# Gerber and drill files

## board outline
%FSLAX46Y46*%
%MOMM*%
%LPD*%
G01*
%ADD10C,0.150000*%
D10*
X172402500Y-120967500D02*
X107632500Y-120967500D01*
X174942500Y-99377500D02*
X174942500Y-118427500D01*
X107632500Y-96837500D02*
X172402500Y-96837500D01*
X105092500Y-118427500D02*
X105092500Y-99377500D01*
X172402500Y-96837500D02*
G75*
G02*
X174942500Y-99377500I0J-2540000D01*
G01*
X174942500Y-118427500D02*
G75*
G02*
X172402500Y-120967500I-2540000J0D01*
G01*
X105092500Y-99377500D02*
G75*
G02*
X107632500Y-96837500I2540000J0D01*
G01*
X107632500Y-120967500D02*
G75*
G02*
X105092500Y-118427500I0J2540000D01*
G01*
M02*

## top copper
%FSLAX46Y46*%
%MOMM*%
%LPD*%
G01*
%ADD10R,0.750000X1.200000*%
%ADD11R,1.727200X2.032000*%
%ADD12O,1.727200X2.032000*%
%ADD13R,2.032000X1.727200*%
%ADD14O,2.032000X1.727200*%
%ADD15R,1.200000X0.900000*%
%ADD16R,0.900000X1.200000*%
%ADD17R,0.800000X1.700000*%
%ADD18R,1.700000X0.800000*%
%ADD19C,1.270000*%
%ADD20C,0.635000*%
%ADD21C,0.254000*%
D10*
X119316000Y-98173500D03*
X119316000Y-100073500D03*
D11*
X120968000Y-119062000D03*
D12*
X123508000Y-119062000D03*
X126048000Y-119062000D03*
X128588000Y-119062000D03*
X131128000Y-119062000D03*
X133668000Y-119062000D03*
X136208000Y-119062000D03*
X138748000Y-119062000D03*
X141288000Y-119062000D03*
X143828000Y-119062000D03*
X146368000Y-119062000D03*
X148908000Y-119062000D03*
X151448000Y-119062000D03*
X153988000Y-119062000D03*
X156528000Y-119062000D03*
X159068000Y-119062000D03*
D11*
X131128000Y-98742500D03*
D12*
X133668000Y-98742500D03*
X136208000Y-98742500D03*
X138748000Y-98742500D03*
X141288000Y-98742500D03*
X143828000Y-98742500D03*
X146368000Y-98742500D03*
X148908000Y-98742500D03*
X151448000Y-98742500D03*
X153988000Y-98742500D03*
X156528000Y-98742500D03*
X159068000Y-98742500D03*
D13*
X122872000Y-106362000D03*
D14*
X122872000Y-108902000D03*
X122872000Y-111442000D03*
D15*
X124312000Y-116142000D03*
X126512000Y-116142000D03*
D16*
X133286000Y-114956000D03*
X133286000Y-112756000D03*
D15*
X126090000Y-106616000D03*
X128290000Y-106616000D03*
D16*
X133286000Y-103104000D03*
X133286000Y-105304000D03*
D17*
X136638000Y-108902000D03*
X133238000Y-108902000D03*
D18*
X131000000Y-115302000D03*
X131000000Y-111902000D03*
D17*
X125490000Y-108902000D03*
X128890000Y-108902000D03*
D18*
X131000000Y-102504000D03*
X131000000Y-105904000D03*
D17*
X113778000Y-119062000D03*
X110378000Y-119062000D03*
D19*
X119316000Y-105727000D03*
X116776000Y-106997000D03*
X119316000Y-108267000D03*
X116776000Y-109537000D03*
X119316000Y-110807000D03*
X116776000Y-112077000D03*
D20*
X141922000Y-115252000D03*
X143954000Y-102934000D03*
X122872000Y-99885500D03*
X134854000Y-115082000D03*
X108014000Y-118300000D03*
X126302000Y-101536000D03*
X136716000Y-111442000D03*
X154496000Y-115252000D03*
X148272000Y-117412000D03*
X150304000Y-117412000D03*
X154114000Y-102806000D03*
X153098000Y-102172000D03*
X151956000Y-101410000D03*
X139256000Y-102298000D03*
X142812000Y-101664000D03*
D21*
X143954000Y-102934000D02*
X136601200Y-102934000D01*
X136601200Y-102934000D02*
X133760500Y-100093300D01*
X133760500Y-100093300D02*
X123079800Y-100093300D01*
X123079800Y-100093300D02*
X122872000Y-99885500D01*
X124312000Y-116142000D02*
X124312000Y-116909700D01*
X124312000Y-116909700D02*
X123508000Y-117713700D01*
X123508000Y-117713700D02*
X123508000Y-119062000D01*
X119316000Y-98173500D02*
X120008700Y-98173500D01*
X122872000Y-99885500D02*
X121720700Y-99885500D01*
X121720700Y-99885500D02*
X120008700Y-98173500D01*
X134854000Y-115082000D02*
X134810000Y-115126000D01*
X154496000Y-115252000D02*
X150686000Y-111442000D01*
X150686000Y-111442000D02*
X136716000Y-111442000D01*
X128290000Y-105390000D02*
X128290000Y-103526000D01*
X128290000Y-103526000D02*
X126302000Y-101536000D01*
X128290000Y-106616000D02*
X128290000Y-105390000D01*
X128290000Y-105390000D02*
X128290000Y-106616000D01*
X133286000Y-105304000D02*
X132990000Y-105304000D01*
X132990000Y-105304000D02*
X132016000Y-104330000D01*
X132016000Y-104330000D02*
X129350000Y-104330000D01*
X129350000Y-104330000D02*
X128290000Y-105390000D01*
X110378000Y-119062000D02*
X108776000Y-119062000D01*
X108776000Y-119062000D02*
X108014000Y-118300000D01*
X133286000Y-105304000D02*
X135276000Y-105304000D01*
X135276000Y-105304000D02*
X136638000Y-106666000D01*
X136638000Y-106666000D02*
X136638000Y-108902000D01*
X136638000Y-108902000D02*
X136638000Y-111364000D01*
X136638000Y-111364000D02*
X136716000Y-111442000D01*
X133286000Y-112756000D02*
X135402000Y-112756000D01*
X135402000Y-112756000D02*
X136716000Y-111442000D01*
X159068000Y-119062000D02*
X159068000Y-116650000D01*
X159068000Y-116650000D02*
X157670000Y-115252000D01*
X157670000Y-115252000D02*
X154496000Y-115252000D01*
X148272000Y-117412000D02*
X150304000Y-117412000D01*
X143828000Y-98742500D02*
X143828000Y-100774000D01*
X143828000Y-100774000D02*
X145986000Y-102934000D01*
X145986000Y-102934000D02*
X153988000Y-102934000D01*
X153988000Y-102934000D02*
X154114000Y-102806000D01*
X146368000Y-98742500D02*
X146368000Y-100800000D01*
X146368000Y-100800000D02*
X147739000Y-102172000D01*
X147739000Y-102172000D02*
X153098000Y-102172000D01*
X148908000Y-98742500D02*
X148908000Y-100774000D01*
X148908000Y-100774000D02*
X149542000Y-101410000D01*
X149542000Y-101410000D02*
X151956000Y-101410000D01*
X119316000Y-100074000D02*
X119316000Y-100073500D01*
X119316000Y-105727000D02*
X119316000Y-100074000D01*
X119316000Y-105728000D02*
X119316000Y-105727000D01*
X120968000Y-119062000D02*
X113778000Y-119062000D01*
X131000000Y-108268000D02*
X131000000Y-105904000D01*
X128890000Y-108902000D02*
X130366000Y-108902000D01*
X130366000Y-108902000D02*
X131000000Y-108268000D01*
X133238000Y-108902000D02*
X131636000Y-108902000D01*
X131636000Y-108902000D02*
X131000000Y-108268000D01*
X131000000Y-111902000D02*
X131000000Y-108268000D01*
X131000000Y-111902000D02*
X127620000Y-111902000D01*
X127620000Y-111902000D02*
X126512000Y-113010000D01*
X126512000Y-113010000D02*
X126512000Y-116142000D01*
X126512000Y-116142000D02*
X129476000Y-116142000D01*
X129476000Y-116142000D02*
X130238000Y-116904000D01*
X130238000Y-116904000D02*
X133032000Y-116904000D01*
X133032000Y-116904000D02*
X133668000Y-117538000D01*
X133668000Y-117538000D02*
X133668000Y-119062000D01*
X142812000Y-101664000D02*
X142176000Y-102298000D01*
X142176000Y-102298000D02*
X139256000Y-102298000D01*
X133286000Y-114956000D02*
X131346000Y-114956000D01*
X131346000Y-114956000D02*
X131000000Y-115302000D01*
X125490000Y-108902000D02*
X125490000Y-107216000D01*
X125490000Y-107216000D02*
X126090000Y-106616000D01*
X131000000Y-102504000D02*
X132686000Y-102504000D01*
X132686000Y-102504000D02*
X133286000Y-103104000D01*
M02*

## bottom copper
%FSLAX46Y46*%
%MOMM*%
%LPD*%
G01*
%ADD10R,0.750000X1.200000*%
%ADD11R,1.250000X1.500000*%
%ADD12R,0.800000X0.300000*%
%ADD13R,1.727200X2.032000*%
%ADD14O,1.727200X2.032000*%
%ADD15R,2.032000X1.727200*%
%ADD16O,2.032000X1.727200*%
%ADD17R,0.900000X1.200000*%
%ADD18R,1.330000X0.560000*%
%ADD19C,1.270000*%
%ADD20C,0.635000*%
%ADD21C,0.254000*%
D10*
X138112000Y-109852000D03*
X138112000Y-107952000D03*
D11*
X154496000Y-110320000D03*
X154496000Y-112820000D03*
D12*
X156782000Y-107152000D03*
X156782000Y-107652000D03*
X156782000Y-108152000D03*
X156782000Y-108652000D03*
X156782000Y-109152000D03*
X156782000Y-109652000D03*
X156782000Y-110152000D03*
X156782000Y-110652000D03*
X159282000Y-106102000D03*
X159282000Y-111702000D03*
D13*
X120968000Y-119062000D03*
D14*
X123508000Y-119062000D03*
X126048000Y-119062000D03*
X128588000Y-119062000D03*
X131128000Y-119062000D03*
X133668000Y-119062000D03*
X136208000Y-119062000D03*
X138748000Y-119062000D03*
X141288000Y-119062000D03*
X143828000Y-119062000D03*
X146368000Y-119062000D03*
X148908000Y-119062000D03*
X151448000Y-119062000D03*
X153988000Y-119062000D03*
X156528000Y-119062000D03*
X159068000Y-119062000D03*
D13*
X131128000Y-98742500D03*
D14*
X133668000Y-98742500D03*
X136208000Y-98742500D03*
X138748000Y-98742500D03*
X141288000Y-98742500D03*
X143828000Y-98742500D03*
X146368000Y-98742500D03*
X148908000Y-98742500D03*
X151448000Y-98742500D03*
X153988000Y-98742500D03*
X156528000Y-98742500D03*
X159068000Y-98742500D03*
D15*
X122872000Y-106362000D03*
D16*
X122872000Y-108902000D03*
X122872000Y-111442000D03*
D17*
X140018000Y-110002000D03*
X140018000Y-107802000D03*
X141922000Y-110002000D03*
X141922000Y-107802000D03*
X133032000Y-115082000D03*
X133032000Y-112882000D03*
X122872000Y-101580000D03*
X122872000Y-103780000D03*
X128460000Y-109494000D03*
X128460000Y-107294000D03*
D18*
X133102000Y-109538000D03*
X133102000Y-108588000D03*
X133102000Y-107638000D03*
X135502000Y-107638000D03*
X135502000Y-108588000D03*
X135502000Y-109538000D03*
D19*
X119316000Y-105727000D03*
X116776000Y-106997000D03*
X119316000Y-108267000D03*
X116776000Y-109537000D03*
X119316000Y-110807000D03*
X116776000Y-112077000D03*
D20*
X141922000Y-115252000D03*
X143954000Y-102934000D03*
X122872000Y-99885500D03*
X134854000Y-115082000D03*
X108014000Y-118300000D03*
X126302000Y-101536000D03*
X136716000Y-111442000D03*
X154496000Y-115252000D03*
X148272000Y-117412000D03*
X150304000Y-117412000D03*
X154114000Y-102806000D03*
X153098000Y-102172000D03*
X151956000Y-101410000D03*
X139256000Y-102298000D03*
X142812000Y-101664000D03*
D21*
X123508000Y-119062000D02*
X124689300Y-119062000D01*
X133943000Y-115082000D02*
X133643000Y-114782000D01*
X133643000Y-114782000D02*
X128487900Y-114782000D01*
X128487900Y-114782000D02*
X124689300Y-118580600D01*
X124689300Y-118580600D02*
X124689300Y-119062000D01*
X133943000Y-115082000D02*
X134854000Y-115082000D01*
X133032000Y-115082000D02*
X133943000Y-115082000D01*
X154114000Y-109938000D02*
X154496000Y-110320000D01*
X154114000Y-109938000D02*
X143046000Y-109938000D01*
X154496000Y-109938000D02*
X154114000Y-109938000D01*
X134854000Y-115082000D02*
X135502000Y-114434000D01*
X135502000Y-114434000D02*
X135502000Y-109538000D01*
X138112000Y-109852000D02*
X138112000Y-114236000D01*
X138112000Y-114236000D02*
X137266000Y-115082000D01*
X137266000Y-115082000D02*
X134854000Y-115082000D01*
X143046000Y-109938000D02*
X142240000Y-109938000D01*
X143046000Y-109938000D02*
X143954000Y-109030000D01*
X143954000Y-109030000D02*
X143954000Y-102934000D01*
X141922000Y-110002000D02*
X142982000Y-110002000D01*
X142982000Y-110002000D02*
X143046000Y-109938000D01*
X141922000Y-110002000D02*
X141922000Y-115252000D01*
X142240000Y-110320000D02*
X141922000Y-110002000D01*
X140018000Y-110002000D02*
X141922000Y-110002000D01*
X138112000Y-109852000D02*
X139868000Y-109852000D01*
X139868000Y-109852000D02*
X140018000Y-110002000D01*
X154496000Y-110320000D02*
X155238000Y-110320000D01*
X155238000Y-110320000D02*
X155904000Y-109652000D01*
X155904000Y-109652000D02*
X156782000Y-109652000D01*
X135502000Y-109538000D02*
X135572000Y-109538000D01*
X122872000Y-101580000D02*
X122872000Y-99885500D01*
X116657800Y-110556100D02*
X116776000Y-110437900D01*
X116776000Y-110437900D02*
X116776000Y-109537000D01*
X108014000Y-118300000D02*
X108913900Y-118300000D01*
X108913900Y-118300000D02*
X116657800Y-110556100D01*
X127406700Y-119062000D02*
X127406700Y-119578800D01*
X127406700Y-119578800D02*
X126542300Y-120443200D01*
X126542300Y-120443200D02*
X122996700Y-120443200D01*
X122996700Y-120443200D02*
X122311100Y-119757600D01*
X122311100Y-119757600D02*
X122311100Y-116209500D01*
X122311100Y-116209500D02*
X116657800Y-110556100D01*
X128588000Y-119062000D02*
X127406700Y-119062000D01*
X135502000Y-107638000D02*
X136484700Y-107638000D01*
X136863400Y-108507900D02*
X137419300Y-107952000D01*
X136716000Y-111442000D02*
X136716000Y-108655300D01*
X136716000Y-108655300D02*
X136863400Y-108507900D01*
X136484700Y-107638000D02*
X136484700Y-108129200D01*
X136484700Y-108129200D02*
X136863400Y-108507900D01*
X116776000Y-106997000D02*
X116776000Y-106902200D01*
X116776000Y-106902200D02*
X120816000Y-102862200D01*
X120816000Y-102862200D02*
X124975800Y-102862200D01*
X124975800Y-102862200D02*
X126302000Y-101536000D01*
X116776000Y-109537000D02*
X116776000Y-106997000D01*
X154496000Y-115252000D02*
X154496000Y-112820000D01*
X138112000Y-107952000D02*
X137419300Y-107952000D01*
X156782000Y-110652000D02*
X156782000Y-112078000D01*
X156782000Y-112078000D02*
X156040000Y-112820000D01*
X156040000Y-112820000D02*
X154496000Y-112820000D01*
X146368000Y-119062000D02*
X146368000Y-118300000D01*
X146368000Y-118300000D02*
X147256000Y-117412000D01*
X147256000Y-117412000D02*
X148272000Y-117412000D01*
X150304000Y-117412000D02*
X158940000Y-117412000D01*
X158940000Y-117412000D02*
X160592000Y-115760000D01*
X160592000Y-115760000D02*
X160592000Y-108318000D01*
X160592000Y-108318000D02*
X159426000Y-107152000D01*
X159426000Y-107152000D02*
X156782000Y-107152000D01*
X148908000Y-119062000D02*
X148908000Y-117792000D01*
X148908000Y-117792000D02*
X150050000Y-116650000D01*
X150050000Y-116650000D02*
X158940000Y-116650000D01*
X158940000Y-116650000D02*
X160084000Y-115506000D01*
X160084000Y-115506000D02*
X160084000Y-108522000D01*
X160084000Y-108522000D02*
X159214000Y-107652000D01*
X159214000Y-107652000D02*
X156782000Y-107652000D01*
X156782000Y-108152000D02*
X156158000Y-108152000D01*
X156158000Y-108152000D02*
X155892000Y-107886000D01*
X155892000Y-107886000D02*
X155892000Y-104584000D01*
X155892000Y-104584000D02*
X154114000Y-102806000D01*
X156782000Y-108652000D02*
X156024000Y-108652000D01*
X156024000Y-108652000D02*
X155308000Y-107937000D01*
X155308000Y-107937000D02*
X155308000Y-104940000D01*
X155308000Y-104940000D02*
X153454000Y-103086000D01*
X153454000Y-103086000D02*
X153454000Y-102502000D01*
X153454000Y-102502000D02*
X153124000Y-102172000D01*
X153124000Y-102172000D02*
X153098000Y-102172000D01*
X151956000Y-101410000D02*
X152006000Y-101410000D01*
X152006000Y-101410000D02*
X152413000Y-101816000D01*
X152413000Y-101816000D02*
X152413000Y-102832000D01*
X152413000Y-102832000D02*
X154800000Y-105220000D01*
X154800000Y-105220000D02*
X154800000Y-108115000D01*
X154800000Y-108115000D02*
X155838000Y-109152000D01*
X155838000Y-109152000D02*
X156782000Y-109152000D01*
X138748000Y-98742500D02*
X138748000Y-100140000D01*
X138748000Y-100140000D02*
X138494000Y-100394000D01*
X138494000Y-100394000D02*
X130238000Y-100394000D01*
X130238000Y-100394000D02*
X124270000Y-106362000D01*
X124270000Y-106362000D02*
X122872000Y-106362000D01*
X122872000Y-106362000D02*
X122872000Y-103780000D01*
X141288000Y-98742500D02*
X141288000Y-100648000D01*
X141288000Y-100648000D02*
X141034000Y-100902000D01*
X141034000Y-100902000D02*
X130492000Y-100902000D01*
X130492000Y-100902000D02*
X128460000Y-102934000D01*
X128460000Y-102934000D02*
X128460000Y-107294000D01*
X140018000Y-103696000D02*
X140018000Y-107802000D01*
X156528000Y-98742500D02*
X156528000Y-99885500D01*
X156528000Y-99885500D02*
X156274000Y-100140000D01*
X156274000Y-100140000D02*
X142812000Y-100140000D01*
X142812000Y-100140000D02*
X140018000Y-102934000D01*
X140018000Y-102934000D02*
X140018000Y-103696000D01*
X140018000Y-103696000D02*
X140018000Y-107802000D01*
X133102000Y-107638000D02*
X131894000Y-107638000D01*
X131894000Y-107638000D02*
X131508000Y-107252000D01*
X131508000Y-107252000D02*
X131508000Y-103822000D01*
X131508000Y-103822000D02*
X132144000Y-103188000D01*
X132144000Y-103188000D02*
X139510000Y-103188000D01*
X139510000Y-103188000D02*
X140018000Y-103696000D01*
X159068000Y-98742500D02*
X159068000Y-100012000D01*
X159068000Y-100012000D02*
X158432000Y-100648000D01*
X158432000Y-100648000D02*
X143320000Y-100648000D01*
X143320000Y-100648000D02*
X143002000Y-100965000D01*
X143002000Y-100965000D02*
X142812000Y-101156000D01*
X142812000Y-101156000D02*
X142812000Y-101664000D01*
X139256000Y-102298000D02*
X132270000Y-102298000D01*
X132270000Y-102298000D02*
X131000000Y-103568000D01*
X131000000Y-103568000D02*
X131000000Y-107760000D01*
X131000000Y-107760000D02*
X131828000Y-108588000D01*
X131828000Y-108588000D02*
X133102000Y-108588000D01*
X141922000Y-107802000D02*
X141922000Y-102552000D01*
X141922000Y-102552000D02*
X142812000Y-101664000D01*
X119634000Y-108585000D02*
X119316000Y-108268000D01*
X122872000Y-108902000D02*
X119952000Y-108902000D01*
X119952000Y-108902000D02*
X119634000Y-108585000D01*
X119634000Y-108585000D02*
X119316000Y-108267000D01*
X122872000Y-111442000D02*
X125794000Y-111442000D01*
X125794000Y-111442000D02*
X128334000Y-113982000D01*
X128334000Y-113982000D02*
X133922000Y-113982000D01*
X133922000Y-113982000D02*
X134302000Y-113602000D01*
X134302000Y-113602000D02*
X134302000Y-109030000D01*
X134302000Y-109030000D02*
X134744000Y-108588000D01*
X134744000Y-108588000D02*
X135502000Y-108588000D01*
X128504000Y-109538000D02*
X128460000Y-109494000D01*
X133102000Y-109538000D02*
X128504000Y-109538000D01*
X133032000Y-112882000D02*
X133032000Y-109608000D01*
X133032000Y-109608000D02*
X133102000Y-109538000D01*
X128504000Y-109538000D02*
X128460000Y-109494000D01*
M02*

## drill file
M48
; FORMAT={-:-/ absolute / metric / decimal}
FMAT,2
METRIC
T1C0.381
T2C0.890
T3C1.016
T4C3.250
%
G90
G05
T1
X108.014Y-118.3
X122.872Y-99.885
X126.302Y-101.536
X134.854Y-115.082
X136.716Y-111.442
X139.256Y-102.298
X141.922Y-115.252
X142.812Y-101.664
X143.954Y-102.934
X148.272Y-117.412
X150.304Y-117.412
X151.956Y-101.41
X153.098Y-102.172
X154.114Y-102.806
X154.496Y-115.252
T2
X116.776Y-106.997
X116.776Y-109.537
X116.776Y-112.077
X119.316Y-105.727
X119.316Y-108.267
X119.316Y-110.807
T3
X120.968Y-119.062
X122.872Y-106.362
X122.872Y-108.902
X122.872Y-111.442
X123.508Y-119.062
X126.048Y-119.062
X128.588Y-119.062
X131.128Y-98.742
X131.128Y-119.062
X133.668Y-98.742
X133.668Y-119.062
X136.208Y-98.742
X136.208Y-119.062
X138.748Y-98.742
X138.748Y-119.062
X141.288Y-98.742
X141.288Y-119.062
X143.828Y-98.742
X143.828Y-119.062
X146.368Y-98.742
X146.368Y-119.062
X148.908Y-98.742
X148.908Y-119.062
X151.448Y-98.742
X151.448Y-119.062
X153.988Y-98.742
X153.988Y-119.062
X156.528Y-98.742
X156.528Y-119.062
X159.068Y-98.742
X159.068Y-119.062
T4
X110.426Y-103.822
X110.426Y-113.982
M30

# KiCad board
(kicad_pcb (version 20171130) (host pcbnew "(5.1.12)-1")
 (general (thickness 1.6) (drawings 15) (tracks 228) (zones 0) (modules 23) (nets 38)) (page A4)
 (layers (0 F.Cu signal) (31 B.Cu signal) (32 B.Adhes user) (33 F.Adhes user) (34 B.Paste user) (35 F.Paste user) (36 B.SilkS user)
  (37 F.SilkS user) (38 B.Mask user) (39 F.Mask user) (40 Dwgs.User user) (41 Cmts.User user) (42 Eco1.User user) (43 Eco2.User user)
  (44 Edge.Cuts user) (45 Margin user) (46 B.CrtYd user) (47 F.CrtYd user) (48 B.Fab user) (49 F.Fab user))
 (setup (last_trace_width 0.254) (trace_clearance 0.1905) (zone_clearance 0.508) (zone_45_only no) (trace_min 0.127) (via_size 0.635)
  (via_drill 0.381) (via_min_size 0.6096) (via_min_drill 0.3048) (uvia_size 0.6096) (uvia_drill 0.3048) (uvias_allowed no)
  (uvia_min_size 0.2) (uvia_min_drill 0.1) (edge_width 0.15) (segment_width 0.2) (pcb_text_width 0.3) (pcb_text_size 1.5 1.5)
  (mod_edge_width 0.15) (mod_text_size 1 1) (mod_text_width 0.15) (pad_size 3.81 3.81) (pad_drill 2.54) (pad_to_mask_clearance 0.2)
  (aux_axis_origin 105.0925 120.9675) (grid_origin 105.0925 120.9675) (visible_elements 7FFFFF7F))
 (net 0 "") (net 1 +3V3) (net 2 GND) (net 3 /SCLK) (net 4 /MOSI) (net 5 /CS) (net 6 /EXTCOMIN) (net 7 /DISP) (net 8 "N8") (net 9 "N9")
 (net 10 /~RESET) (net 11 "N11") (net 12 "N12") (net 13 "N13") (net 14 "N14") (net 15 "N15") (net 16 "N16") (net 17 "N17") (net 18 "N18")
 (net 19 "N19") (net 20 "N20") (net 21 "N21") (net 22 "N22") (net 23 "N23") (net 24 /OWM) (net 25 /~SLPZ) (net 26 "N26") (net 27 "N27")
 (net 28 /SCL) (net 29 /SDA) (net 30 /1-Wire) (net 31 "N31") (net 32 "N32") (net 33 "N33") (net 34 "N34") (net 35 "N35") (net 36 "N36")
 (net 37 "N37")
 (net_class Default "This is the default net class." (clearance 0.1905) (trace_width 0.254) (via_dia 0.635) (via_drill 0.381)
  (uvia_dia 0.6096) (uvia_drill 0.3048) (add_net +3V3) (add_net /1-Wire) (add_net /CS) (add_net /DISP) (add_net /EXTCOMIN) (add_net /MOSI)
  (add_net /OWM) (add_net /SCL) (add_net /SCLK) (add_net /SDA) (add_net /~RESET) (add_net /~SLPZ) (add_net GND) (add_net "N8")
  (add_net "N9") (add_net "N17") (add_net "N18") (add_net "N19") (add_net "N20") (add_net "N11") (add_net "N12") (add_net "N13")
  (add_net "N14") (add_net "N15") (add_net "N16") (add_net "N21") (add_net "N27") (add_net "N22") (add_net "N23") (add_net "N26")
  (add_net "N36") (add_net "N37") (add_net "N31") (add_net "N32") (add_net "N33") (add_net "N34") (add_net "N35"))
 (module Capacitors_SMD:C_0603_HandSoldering (layer B.Cu) (at 138.112 108.902 90)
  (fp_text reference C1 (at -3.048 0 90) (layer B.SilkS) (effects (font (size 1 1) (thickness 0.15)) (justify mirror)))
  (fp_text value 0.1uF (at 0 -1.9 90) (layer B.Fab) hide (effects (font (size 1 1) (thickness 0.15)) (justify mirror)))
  (pad 1 smd rect (at -0.95 0 90) (size 1.2 0.75) (layers B.Cu B.Paste B.Mask) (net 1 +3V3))
  (pad 2 smd rect (at 0.95 0 90) (size 1.2 0.75) (layers B.Cu B.Paste B.Mask) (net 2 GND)))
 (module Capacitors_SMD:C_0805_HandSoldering (layer B.Cu) (at 154.496 111.57 270)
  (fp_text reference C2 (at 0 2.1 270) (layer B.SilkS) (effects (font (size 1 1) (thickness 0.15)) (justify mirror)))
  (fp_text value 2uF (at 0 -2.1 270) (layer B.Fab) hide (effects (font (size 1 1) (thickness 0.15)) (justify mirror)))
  (pad 1 smd rect (at -1.25 0 270) (size 1.5 1.25) (layers B.Cu B.Paste B.Mask) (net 1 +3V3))
  (pad 2 smd rect (at 1.25 0 270) (size 1.5 1.25) (layers B.Cu B.Paste B.Mask) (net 2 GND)))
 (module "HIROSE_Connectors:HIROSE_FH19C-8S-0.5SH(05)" (layer B.Cu) (at 156.782 108.902 270)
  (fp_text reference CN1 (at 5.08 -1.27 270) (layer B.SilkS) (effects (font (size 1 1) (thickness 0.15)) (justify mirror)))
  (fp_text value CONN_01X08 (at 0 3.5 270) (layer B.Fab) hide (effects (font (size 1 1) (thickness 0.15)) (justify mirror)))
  (pad 1 smd rect (at -1.75 0 270) (size 0.3 0.8) (layers B.Cu B.Paste B.Mask) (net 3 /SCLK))
  (pad 2 smd rect (at -1.25 0 270) (size 0.3 0.8) (layers B.Cu B.Paste B.Mask) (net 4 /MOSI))
  (pad 3 smd rect (at -0.75 0 270) (size 0.3 0.8) (layers B.Cu B.Paste B.Mask) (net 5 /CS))
  (pad 4 smd rect (at -0.25 0 270) (size 0.3 0.8) (layers B.Cu B.Paste B.Mask) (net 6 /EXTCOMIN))
  (pad 5 smd rect (at 0.25 0 270) (size 0.3 0.8) (layers B.Cu B.Paste B.Mask) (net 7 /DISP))
  (pad 6 smd rect (at 0.75 0 270) (size 0.3 0.8) (layers B.Cu B.Paste B.Mask) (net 1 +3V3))
  (pad 7 smd rect (at 1.25 0 270) (size 0.3 0.8) (layers B.Cu B.Paste B.Mask) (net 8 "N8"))
  (pad 8 smd rect (at 1.75 0 270) (size 0.3 0.8) (layers B.Cu B.Paste B.Mask) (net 2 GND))
  (pad "" smd rect (at -2.8 -2.5 270) (size 0.3 0.8) (layers B.Cu B.Paste B.Mask))
  (pad "" smd rect (at 2.8 -2.5 270) (size 0.3 0.8) (layers B.Cu B.Paste B.Mask)))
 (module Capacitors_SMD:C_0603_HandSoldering (layer F.Cu) (at 119.316 99.1235 270)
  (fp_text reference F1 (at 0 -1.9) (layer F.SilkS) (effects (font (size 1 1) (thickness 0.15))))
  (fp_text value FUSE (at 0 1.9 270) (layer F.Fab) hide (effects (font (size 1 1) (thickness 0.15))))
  (pad 1 smd rect (at -0.95 0 270) (size 1.2 0.75) (layers F.Cu F.Paste F.Mask) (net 1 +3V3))
  (pad 2 smd rect (at 0.95 0 270) (size 1.2 0.75) (layers F.Cu F.Paste F.Mask) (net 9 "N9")))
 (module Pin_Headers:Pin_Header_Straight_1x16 (layer B.Cu) (at 120.968 119.062 270)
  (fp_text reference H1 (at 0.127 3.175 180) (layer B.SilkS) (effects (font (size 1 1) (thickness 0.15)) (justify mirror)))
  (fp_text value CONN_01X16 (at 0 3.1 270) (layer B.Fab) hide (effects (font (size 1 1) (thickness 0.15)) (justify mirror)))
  (pad 1 thru_hole rect (at 0 0 270) (size 2.032 1.7272) (drill 1.016) (layers *.Cu *.Mask B.SilkS) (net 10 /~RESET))
  (pad 2 thru_hole oval (at 0 -2.54 270) (size 2.032 1.7272) (drill 1.016) (layers *.Cu *.Mask B.SilkS) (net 1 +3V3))
  (pad 3 thru_hole oval (at 0 -5.08 270) (size 2.032 1.7272) (drill 1.016) (layers *.Cu *.Mask B.SilkS) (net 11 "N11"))
  (pad 4 thru_hole oval (at 0 -7.62 270) (size 2.032 1.7272) (drill 1.016) (layers *.Cu *.Mask B.SilkS) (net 2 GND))
  (pad 5 thru_hole oval (at 0 -10.16 270) (size 2.032 1.7272) (drill 1.016) (layers *.Cu *.Mask B.SilkS) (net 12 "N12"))
  (pad 6 thru_hole oval (at 0 -12.7 270) (size 2.032 1.7272) (drill 1.016) (layers *.Cu *.Mask B.SilkS) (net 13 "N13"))
  (pad 7 thru_hole oval (at 0 -15.24 270) (size 2.032 1.7272) (drill 1.016) (layers *.Cu *.Mask B.SilkS) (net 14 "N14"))
  (pad 8 thru_hole oval (at 0 -17.78 270) (size 2.032 1.7272) (drill 1.016) (layers *.Cu *.Mask B.SilkS) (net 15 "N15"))
  (pad 9 thru_hole oval (at 0 -20.32 270) (size 2.032 1.7272) (drill 1.016) (layers *.Cu *.Mask B.SilkS) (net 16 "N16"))
  (pad 10 thru_hole oval (at 0 -22.86 270) (size 2.032 1.7272) (drill 1.016) (layers *.Cu *.Mask B.SilkS) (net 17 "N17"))
  (pad 11 thru_hole oval (at 0 -25.4 270) (size 2.032 1.7272) (drill 1.016) (layers *.Cu *.Mask B.SilkS) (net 3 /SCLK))
  (pad 12 thru_hole oval (at 0 -27.94 270) (size 2.032 1.7272) (drill 1.016) (layers *.Cu *.Mask B.SilkS) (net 4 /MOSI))
  (pad 13 thru_hole oval (at 0 -30.48 270) (size 2.032 1.7272) (drill 1.016) (layers *.Cu *.Mask B.SilkS) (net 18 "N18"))
  (pad 14 thru_hole oval (at 0 -33.02 270) (size 2.032 1.7272) (drill 1.016) (layers *.Cu *.Mask B.SilkS) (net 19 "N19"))
  (pad 15 thru_hole oval (at 0 -35.56 270) (size 2.032 1.7272) (drill 1.016) (layers *.Cu *.Mask B.SilkS) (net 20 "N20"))
  (pad 16 thru_hole oval (at 0 -38.1 270) (size 2.032 1.7272) (drill 1.016) (layers *.Cu *.Mask B.SilkS) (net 2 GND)))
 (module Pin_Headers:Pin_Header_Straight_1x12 (layer B.Cu) (at 131.128 98.7425 270)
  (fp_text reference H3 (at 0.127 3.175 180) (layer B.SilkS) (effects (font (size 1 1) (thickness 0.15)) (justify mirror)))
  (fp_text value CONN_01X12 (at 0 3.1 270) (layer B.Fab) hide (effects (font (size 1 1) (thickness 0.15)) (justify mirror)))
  (pad 1 thru_hole rect (at 0 0 270) (size 2.032 1.7272) (drill 1.016) (layers *.Cu *.Mask B.SilkS) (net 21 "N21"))
  (pad 2 thru_hole oval (at 0 -2.54 270) (size 2.032 1.7272) (drill 1.016) (layers *.Cu *.Mask B.SilkS) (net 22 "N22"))
  (pad 3 thru_hole oval (at 0 -5.08 270) (size 2.032 1.7272) (drill 1.016) (layers *.Cu *.Mask B.SilkS) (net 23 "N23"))
  (pad 4 thru_hole oval (at 0 -7.62 270) (size 2.032 1.7272) (drill 1.016) (layers *.Cu *.Mask B.SilkS) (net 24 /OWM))
  (pad 5 thru_hole oval (at 0 -10.16 270) (size 2.032 1.7272) (drill 1.016) (layers *.Cu *.Mask B.SilkS) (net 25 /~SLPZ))
  (pad 6 thru_hole oval (at 0 -12.7 270) (size 2.032 1.7272) (drill 1.016) (layers *.Cu *.Mask B.SilkS) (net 5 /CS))
  (pad 7 thru_hole oval (at 0 -15.24 270) (size 2.032 1.7272) (drill 1.016) (layers *.Cu *.Mask B.SilkS) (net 6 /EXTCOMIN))
  (pad 8 thru_hole oval (at 0 -17.78 270) (size 2.032 1.7272) (drill 1.016) (layers *.Cu *.Mask B.SilkS) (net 7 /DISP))
  (pad 9 thru_hole oval (at 0 -20.32 270) (size 2.032 1.7272) (drill 1.016) (layers *.Cu *.Mask B.SilkS) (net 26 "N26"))
  (pad 10 thru_hole oval (at 0 -22.86 270) (size 2.032 1.7272) (drill 1.016) (layers *.Cu *.Mask B.SilkS) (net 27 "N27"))
  (pad 11 thru_hole oval (at 0 -25.4 270) (size 2.032 1.7272) (drill 1.016) (layers *.Cu *.Mask B.SilkS) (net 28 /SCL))
  (pad 12 thru_hole oval (at 0 -27.94 270) (size 2.032 1.7272) (drill 1.016) (layers *.Cu *.Mask B.SilkS) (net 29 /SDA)))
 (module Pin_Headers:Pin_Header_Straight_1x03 (layer F.Cu) (at 122.872 106.362)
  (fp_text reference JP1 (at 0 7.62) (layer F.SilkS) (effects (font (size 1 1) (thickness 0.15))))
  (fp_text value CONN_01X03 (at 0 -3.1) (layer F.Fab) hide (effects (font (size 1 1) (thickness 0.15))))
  (pad 1 thru_hole rect (at 0 0) (size 2.032 1.7272) (drill 1.016) (layers *.Cu *.Mask F.SilkS) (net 24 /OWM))
  (pad 2 thru_hole oval (at 0 2.54) (size 2.032 1.7272) (drill 1.016) (layers *.Cu *.Mask F.SilkS) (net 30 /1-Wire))
  (pad 3 thru_hole oval (at 0 5.08) (size 2.032 1.7272) (drill 1.016) (layers *.Cu *.Mask F.SilkS) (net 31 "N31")))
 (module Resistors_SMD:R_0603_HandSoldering (layer B.Cu) (at 140.018 108.902 90)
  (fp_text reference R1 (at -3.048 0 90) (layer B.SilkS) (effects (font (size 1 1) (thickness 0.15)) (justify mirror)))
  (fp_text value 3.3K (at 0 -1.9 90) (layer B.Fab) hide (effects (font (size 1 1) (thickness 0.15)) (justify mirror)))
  (pad 1 smd rect (at -1.1 0 90) (size 1.2 0.9) (layers B.Cu B.Paste B.Mask) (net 1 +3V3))
  (pad 2 smd rect (at 1.1 0 90) (size 1.2 0.9) (layers B.Cu B.Paste B.Mask) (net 28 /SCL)))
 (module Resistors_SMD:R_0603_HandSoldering (layer B.Cu) (at 141.922 108.902 90)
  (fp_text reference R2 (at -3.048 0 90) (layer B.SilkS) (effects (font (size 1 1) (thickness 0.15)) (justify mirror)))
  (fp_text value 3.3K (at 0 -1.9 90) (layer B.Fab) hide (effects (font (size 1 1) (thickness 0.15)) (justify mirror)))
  (pad 1 smd rect (at -1.1 0 90) (size 1.2 0.9) (layers B.Cu B.Paste B.Mask) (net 1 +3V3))
  (pad 2 smd rect (at 1.1 0 90) (size 1.2 0.9) (layers B.Cu B.Paste B.Mask) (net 29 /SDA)))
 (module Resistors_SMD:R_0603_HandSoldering (layer B.Cu) (at 133.032 113.982 90)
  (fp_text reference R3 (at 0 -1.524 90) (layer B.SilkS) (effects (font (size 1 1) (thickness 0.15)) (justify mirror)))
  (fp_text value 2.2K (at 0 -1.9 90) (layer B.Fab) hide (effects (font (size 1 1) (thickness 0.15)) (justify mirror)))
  (pad 1 smd rect (at -1.1 0 90) (size 1.2 0.9) (layers B.Cu B.Paste B.Mask) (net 1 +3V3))
  (pad 2 smd rect (at 1.1 0 90) (size 1.2 0.9) (layers B.Cu B.Paste B.Mask) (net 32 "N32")))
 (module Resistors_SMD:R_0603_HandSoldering (layer B.Cu) (at 122.872 102.68 270)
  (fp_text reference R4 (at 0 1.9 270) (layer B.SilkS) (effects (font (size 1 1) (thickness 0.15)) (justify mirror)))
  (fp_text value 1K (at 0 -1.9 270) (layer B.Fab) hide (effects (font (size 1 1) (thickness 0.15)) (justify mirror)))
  (pad 1 smd rect (at -1.1 0 270) (size 1.2 0.9) (layers B.Cu B.Paste B.Mask) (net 1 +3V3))
  (pad 2 smd rect (at 1.1 0 270) (size 1.2 0.9) (layers B.Cu B.Paste B.Mask) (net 24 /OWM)))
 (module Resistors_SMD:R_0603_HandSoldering (layer B.Cu) (at 128.46 108.394 90)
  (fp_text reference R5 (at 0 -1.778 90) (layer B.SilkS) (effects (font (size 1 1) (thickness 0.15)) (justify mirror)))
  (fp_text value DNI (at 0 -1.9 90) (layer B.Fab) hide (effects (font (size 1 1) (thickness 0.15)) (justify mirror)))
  (pad 1 smd rect (at -1.1 0 90) (size 1.2 0.9) (layers B.Cu B.Paste B.Mask) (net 32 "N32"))
  (pad 2 smd rect (at 1.1 0 90) (size 1.2 0.9) (layers B.Cu B.Paste B.Mask) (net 25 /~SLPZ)))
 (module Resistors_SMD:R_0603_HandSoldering (layer F.Cu) (at 125.412 116.142)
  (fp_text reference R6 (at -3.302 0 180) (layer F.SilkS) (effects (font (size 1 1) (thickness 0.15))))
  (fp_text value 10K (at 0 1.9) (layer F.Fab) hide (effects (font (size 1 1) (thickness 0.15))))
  (pad 1 smd rect (at -1.1 0) (size 1.2 0.9) (layers F.Cu F.Paste F.Mask) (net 1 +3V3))
  (pad 2 smd rect (at 1.1 0) (size 1.2 0.9) (layers F.Cu F.Paste F.Mask) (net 13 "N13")))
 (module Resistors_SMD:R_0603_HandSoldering (layer F.Cu) (at 133.286 113.856 90)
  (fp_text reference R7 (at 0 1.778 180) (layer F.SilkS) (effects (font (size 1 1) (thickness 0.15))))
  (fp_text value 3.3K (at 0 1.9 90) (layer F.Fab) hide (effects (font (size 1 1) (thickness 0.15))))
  (pad 1 smd rect (at -1.1 0 90) (size 1.2 0.9) (layers F.Cu F.Paste F.Mask) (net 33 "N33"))
  (pad 2 smd rect (at 1.1 0 90) (size 1.2 0.9) (layers F.Cu F.Paste F.Mask) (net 2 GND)))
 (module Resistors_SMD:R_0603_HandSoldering (layer F.Cu) (at 127.19 106.616)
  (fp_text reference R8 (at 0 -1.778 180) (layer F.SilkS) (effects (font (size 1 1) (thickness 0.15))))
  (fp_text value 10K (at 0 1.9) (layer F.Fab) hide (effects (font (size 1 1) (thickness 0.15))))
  (pad 1 smd rect (at -1.1 0) (size 1.2 0.9) (layers F.Cu F.Paste F.Mask) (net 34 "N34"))
  (pad 2 smd rect (at 1.1 0) (size 1.2 0.9) (layers F.Cu F.Paste F.Mask) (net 2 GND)))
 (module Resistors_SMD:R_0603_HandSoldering (layer F.Cu) (at 133.286 104.204 270)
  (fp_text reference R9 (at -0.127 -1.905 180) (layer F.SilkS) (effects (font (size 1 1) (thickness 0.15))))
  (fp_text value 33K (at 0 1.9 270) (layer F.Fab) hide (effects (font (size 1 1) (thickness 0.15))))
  (pad 1 smd rect (at -1.1 0 270) (size 1.2 0.9) (layers F.Cu F.Paste F.Mask) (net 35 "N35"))
  (pad 2 smd rect (at 1.1 0 270) (size 1.2 0.9) (layers F.Cu F.Paste F.Mask) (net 2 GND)))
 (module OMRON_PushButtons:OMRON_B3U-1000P (layer F.Cu) (at 134.938 108.902 180)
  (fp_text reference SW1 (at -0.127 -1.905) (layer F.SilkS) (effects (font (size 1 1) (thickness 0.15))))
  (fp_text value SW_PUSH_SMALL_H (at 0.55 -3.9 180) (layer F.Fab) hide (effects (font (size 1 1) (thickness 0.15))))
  (pad 1 smd rect (at -1.7 0 180) (size 0.8 1.7) (layers F.Cu F.Paste F.Mask) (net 2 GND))
  (pad 2 smd rect (at 1.7 0 180) (size 0.8 1.7) (layers F.Cu F.Paste F.Mask) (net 13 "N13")))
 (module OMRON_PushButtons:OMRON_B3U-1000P (layer F.Cu) (at 131 113.602 90)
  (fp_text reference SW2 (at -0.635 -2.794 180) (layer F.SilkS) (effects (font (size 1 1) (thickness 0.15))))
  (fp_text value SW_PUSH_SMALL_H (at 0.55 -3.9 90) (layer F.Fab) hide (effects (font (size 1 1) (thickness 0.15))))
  (pad 1 smd rect (at -1.7 0 90) (size 0.8 1.7) (layers F.Cu F.Paste F.Mask) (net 33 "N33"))
  (pad 2 smd rect (at 1.7 0 90) (size 0.8 1.7) (layers F.Cu F.Paste F.Mask) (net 13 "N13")))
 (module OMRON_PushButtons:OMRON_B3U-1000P (layer F.Cu) (at 127.19 108.902)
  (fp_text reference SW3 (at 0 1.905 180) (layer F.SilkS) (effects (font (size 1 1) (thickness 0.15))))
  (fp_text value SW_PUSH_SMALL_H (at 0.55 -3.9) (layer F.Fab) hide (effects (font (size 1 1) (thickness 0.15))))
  (pad 1 smd rect (at -1.7 0) (size 0.8 1.7) (layers F.Cu F.Paste F.Mask) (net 34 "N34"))
  (pad 2 smd rect (at 1.7 0) (size 0.8 1.7) (layers F.Cu F.Paste F.Mask) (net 13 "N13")))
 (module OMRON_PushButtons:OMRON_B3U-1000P (layer F.Cu) (at 131 104.204 270)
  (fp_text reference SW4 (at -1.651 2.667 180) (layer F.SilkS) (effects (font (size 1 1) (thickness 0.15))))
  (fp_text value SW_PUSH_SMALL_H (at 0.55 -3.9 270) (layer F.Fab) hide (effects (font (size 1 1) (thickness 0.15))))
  (pad 1 smd rect (at -1.7 0 270) (size 0.8 1.7) (layers F.Cu F.Paste F.Mask) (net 35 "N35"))
  (pad 2 smd rect (at 1.7 0 270) (size 0.8 1.7) (layers F.Cu F.Paste F.Mask) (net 13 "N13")))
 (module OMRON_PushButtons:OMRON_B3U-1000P (layer F.Cu) (at 112.078 119.062 180)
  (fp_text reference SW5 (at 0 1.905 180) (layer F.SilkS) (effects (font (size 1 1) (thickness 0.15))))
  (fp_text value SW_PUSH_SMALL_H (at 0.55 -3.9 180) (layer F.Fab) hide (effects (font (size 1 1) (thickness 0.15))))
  (pad 1 smd rect (at -1.7 0 180) (size 0.8 1.7) (layers F.Cu F.Paste F.Mask) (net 10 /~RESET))
  (pad 2 smd rect (at 1.7 0 180) (size 0.8 1.7) (layers F.Cu F.Paste F.Mask) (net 2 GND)))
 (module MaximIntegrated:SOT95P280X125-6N (layer B.Cu) (at 134.302 109.538)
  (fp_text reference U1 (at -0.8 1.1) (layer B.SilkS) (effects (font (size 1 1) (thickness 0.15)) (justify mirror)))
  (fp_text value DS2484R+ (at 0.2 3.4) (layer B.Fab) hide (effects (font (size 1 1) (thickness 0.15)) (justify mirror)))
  (pad 1 smd rect (at -1.2 0) (size 1.33 0.56) (layers B.Cu B.Paste B.Mask) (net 32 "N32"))
  (pad 2 smd rect (at -1.2 -0.95) (size 1.33 0.56) (layers B.Cu B.Paste B.Mask) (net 29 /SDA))
  (pad 3 smd rect (at -1.2 -1.9) (size 1.33 0.56) (layers B.Cu B.Paste B.Mask) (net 28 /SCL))
  (pad 4 smd rect (at 1.2 -1.9) (size 1.33 0.56) (layers B.Cu B.Paste B.Mask) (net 2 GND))
  (pad 5 smd rect (at 1.2 -0.95) (size 1.33 0.56) (layers B.Cu B.Paste B.Mask) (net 31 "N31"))
  (pad 6 smd rect (at 1.2 0) (size 1.33 0.56) (layers B.Cu B.Paste B.Mask) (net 1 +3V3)))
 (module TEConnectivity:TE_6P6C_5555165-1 (layer F.Cu) (at 119.316 108.902 270)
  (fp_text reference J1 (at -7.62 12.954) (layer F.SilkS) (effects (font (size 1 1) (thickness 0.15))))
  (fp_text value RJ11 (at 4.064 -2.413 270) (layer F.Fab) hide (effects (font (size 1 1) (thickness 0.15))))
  (pad 1 thru_hole circle (at -3.175 0 270) (size 1.27 1.27) (drill 0.89) (layers *.Cu *.Mask) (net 9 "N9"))
  (pad 2 thru_hole circle (at -1.905 2.54 270) (size 1.27 1.27) (drill 0.89) (layers *.Cu *.Mask) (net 2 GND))
  (pad 3 thru_hole circle (at -0.635 0 270) (size 1.27 1.27) (drill 0.89) (layers *.Cu *.Mask) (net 30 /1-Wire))
  (pad 4 thru_hole circle (at 0.635 2.54 270) (size 1.27 1.27) (drill 0.89) (layers *.Cu *.Mask) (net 2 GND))
  (pad 5 thru_hole circle (at 1.905 0 270) (size 1.27 1.27) (drill 0.89) (layers *.Cu *.Mask) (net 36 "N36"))
  (pad 6 thru_hole circle (at 3.175 2.54 270) (size 1.27 1.27) (drill 0.89) (layers *.Cu *.Mask) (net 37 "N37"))
  (pad "" np_thru_hole circle (at -5.08 8.89 270) (size 3.25 3.25) (drill 3.25) (layers *.Cu *.Mask))
  (pad "" np_thru_hole circle (at 5.08 8.89 270) (size 3.25 3.25) (drill 3.25) (layers *.Cu *.Mask)))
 (gr_line (start 172.4025 120.9675) (end 107.6325 120.9675) (angle 90) (layer Edge.Cuts) (width 0.15))
 (gr_line (start 174.9425 99.3775) (end 174.9425 118.4275) (angle 90) (layer Edge.Cuts) (width 0.15))
 (gr_line (start 107.6325 96.8375) (end 172.4025 96.8375) (angle 90) (layer Edge.Cuts) (width 0.15))
 (gr_line (start 105.0925 118.4275) (end 105.0925 99.3775) (angle 90) (layer Edge.Cuts) (width 0.15))
 (gr_arc (start 172.4025 99.3775) (end 172.4025 96.8375) (angle 90) (layer Edge.Cuts) (width 0.15))
 (gr_arc (start 172.4025 118.4275) (end 174.9425 118.4275) (angle 90) (layer Edge.Cuts) (width 0.15))
 (gr_arc (start 107.6325 99.3775) (end 105.0925 99.3775) (angle 90) (layer Edge.Cuts) (width 0.15))
 (gr_arc (start 107.6325 118.4275) (end 107.6325 120.9675) (angle 90) (layer Edge.Cuts) (width 0.15))
 (segment (start 143.954 102.934) (end 136.6012 102.934) (width 0.254) (layer F.Cu) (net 1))
 (segment (start 136.6012 102.934) (end 133.7605 100.0933) (width 0.254) (layer F.Cu) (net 1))
 (segment (start 133.7605 100.0933) (end 123.0798 100.0933) (width 0.254) (layer F.Cu) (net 1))
 (segment (start 123.0798 100.0933) (end 122.872 99.8855) (width 0.254) (layer F.Cu) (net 1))
 (segment (start 124.312 116.142) (end 124.312 116.9097) (width 0.254) (layer F.Cu) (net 1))
 (segment (start 124.312 116.9097) (end 123.508 117.7137) (width 0.254) (layer F.Cu) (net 1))
 (segment (start 123.508 117.7137) (end 123.508 119.062) (width 0.254) (layer F.Cu) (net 1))
 (segment (start 123.508 119.062) (end 124.6893 119.062) (width 0.254) (layer B.Cu) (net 1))
 (segment (start 133.943 115.082) (end 133.643 114.782) (width 0.254) (layer B.Cu) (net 1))
 (segment (start 133.643 114.782) (end 128.4879 114.782) (width 0.254) (layer B.Cu) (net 1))
 (segment (start 128.4879 114.782) (end 124.6893 118.5806) (width 0.254) (layer B.Cu) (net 1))
 (segment (start 124.6893 118.5806) (end 124.6893 119.062) (width 0.254) (layer B.Cu) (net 1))
 (segment (start 133.943 115.082) (end 134.854 115.082) (width 0.254) (layer B.Cu) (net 1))
 (segment (start 133.032 115.082) (end 133.943 115.082) (width 0.254) (layer B.Cu) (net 1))
 (segment (start 119.316 98.1735) (end 120.0087 98.1735) (width 0.254) (layer F.Cu) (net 1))
 (segment (start 122.872 99.8855) (end 121.7207 99.8855) (width 0.254) (layer F.Cu) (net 1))
 (segment (start 121.7207 99.8855) (end 120.0087 98.1735) (width 0.254) (layer F.Cu) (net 1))
 (segment (start 154.114 109.938) (end 154.496 110.32) (width 0.254) (layer B.Cu) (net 1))
 (segment (start 154.114 109.938) (end 143.046 109.938) (width 0.254) (layer B.Cu) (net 1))
 (segment (start 154.496 109.938) (end 154.114 109.938) (width 0.254) (layer B.Cu) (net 1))
 (segment (start 134.854 115.082) (end 135.502 114.434) (width 0.254) (layer B.Cu) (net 1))
 (segment (start 135.502 114.434) (end 135.502 109.538) (width 0.254) (layer B.Cu) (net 1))
 (segment (start 138.112 109.852) (end 138.112 114.236) (width 0.254) (layer B.Cu) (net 1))
 (segment (start 138.112 114.236) (end 137.266 115.082) (width 0.254) (layer B.Cu) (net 1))
 (segment (start 137.266 115.082) (end 134.854 115.082) (width 0.254) (layer B.Cu) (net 1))
 (segment (start 143.046 109.938) (end 142.24 109.938) (width 0.254) (layer B.Cu) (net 1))
 (segment (start 143.046 109.938) (end 143.954 109.03) (width 0.254) (layer B.Cu) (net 1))
 (segment (start 143.954 109.03) (end 143.954 102.934) (width 0.254) (layer B.Cu) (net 1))
 (segment (start 141.922 110.002) (end 142.982 110.002) (width 0.254) (layer B.Cu) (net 1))
 (segment (start 142.982 110.002) (end 143.046 109.938) (width 0.254) (layer B.Cu) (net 1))
 (segment (start 141.922 110.002) (end 141.922 115.252) (width 0.254) (layer B.Cu) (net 1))
 (segment (start 142.24 110.32) (end 141.922 110.002) (width 0.254) (layer B.Cu) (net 1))
 (segment (start 140.018 110.002) (end 141.922 110.002) (width 0.254) (layer B.Cu) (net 1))
 (segment (start 138.112 109.852) (end 139.868 109.852) (width 0.254) (layer B.Cu) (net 1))
 (segment (start 139.868 109.852) (end 140.018 110.002) (width 0.254) (layer B.Cu) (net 1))
 (segment (start 154.496 110.32) (end 155.238 110.32) (width 0.254) (layer B.Cu) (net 1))
 (segment (start 155.238 110.32) (end 155.904 109.652) (width 0.254) (layer B.Cu) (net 1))
 (segment (start 155.904 109.652) (end 156.782 109.652) (width 0.254) (layer B.Cu) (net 1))
 (segment (start 135.502 109.538) (end 135.572 109.538) (width 0.254) (layer B.Cu) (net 1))
 (segment (start 122.872 101.58) (end 122.872 99.8855) (width 0.254) (layer B.Cu) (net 1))
 (segment (start 134.854 115.082) (end 134.81 115.126) (width 0.254) (layer F.Cu) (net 1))
 (via (at 141.922 115.252) (size 0.635) (layers F.Cu B.Cu) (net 1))
 (via (at 143.954 102.934) (size 0.635) (layers F.Cu B.Cu) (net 1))
 (via (at 122.872 99.8855) (size 0.635) (layers F.Cu B.Cu) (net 1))
 (via (at 134.854 115.082) (size 0.635) (layers F.Cu B.Cu) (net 1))
 (segment (start 116.6578 110.5561) (end 116.776 110.4379) (width 0.254) (layer B.Cu) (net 2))
 (segment (start 116.776 110.4379) (end 116.776 109.537) (width 0.254) (layer B.Cu) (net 2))
 (segment (start 108.014 118.3) (end 108.9139 118.3) (width 0.254) (layer B.Cu) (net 2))
 (segment (start 108.9139 118.3) (end 116.6578 110.5561) (width 0.254) (layer B.Cu) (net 2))
 (segment (start 127.4067 119.062) (end 127.4067 119.5788) (width 0.254) (layer B.Cu) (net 2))
 (segment (start 127.4067 119.5788) (end 126.5423 120.4432) (width 0.254) (layer B.Cu) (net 2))
 (segment (start 126.5423 120.4432) (end 122.9967 120.4432) (width 0.254) (layer B.Cu) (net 2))
 (segment (start 122.9967 120.4432) (end 122.3111 119.7576) (width 0.254) (layer B.Cu) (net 2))
 (segment (start 122.3111 119.7576) (end 122.3111 116.2095) (width 0.254) (layer B.Cu) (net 2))
 (segment (start 122.3111 116.2095) (end 116.6578 110.5561) (width 0.254) (layer B.Cu) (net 2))
 (segment (start 128.588 119.062) (end 127.4067 119.062) (width 0.254) (layer B.Cu) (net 2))
 (segment (start 135.502 107.638) (end 136.4847 107.638) (width 0.254) (layer B.Cu) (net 2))
 (segment (start 136.8634 108.5079) (end 137.4193 107.952) (width 0.254) (layer B.Cu) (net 2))
 (segment (start 136.716 111.442) (end 136.716 108.6553) (width 0.254) (layer B.Cu) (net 2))
 (segment (start 136.716 108.6553) (end 136.8634 108.5079) (width 0.254) (layer B.Cu) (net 2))
 (segment (start 136.4847 107.638) (end 136.4847 108.1292) (width 0.254) (layer B.Cu) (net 2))
 (segment (start 136.4847 108.1292) (end 136.8634 108.5079) (width 0.254) (layer B.Cu) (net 2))
 (segment (start 116.776 106.997) (end 116.776 106.9022) (width 0.254) (layer B.Cu) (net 2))
 (segment (start 116.776 106.9022) (end 120.816 102.8622) (width 0.254) (layer B.Cu) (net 2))
 (segment (start 120.816 102.8622) (end 124.9758 102.8622) (width 0.254) (layer B.Cu) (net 2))
 (segment (start 124.9758 102.8622) (end 126.302 101.536) (width 0.254) (layer B.Cu) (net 2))
 (segment (start 116.776 109.537) (end 116.776 106.997) (width 0.254) (layer B.Cu) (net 2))
 (segment (start 154.496 115.252) (end 150.686 111.442) (width 0.254) (layer F.Cu) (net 2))
 (segment (start 150.686 111.442) (end 136.716 111.442) (width 0.254) (layer F.Cu) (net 2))
 (segment (start 154.496 115.252) (end 154.496 112.82) (width 0.254) (layer B.Cu) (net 2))
 (segment (start 138.112 107.952) (end 137.4193 107.952) (width 0.254) (layer B.Cu) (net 2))
 (segment (start 128.29 105.39) (end 128.29 103.526) (width 0.254) (layer F.Cu) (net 2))
 (segment (start 128.29 103.526) (end 126.302 101.536) (width 0.254) (layer F.Cu) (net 2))
 (segment (start 128.29 106.616) (end 128.29 105.39) (width 0.254) (layer F.Cu) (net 2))
 (segment (start 128.29 105.39) (end 128.29 106.616) (width 0.254) (layer F.Cu) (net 2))
 (segment (start 133.286 105.304) (end 132.99 105.304) (width 0.254) (layer F.Cu) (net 2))
 (segment (start 132.99 105.304) (end 132.016 104.33) (width 0.254) (layer F.Cu) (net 2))
 (segment (start 132.016 104.33) (end 129.35 104.33) (width 0.254) (layer F.Cu) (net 2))
 (segment (start 129.35 104.33) (end 128.29 105.39) (width 0.254) (layer F.Cu) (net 2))
 (segment (start 110.378 119.062) (end 108.776 119.062) (width 0.254) (layer F.Cu) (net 2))
 (segment (start 108.776 119.062) (end 108.014 118.3) (width 0.254) (layer F.Cu) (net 2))
 (segment (start 156.782 110.652) (end 156.782 112.078) (width 0.254) (layer B.Cu) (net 2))
 (segment (start 156.782 112.078) (end 156.04 112.82) (width 0.254) (layer B.Cu) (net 2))
 (segment (start 156.04 112.82) (end 154.496 112.82) (width 0.254) (layer B.Cu) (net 2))
 (segment (start 133.286 105.304) (end 135.276 105.304) (width 0.254) (layer F.Cu) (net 2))
 (segment (start 135.276 105.304) (end 136.638 106.666) (width 0.254) (layer F.Cu) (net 2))
 (segment (start 136.638 106.666) (end 136.638 108.902) (width 0.254) (layer F.Cu) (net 2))
 (segment (start 136.638 108.902) (end 136.638 111.364) (width 0.254) (layer F.Cu) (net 2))
 (segment (start 136.638 111.364) (end 136.716 111.442) (width 0.254) (layer F.Cu) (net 2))
 (segment (start 133.286 112.756) (end 135.402 112.756) (width 0.254) (layer F.Cu) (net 2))
 (segment (start 135.402 112.756) (end 136.716 111.442) (width 0.254) (layer F.Cu) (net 2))
 (segment (start 159.068 119.062) (end 159.068 116.65) (width 0.254) (layer F.Cu) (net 2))
 (segment (start 159.068 116.65) (end 157.67 115.252) (width 0.254) (layer F.Cu) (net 2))
 (segment (start 157.67 115.252) (end 154.496 115.252) (width 0.254) (layer F.Cu) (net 2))
 (via (at 108.014 118.3) (size 0.635) (layers F.Cu B.Cu) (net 2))
 (via (at 126.302 101.536) (size 0.635) (layers F.Cu B.Cu) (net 2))
 (via (at 136.716 111.442) (size 0.635) (layers F.Cu B.Cu) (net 2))
 (via (at 154.496 115.252) (size 0.635) (layers F.Cu B.Cu) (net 2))
 (segment (start 146.368 119.062) (end 146.368 118.3) (width 0.254) (layer B.Cu) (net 3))
 (segment (start 146.368 118.3) (end 147.256 117.412) (width 0.254) (layer B.Cu) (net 3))
 (segment (start 147.256 117.412) (end 148.272 117.412) (width 0.254) (layer B.Cu) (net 3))
 (segment (start 148.272 117.412) (end 150.304 117.412) (width 0.254) (layer F.Cu) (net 3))
 (segment (start 150.304 117.412) (end 158.94 117.412) (width 0.254) (layer B.Cu) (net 3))
 (segment (start 158.94 117.412) (end 160.592 115.76) (width 0.254) (layer B.Cu) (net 3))
 (segment (start 160.592 115.76) (end 160.592 108.318) (width 0.254) (layer B.Cu) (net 3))
 (segment (start 160.592 108.318) (end 159.426 107.152) (width 0.254) (layer B.Cu) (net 3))
 (segment (start 159.426 107.152) (end 156.782 107.152) (width 0.254) (layer B.Cu) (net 3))
 (via (at 148.272 117.412) (size 0.635) (layers F.Cu B.Cu) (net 3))
 (via (at 150.304 117.412) (size 0.635) (layers F.Cu B.Cu) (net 3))
 (segment (start 148.908 119.062) (end 148.908 117.792) (width 0.254) (layer B.Cu) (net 4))
 (segment (start 148.908 117.792) (end 150.05 116.65) (width 0.254) (layer B.Cu) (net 4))
 (segment (start 150.05 116.65) (end 158.94 116.65) (width 0.254) (layer B.Cu) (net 4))
 (segment (start 158.94 116.65) (end 160.084 115.506) (width 0.254) (layer B.Cu) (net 4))
 (segment (start 160.084 115.506) (end 160.084 108.522) (width 0.254) (layer B.Cu) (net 4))
 (segment (start 160.084 108.522) (end 159.214 107.652) (width 0.254) (layer B.Cu) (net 4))
 (segment (start 159.214 107.652) (end 156.782 107.652) (width 0.254) (layer B.Cu) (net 4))
 (segment (start 143.828 98.7425) (end 143.828 100.774) (width 0.254) (layer F.Cu) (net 5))
 (segment (start 143.828 100.774) (end 145.986 102.934) (width 0.254) (layer F.Cu) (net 5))
 (segment (start 145.986 102.934) (end 153.988 102.934) (width 0.254) (layer F.Cu) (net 5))
 (segment (start 153.988 102.934) (end 154.114 102.806) (width 0.254) (layer F.Cu) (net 5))
 (segment (start 156.782 108.152) (end 156.158 108.152) (width 0.254) (layer B.Cu) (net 5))
 (segment (start 156.158 108.152) (end 155.892 107.886) (width 0.254) (layer B.Cu) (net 5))
 (segment (start 155.892 107.886) (end 155.892 104.584) (width 0.254) (layer B.Cu) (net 5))
 (segment (start 155.892 104.584) (end 154.114 102.806) (width 0.254) (layer B.Cu) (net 5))
 (via (at 154.114 102.806) (size 0.635) (layers F.Cu B.Cu) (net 5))
 (segment (start 146.368 98.7425) (end 146.368 100.8) (width 0.254) (layer F.Cu) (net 6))
 (segment (start 146.368 100.8) (end 147.739 102.172) (width 0.254) (layer F.Cu) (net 6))
 (segment (start 147.739 102.172) (end 153.098 102.172) (width 0.254) (layer F.Cu) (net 6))
 (segment (start 156.782 108.652) (end 156.024 108.652) (width 0.254) (layer B.Cu) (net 6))
 (segment (start 156.024 108.652) (end 155.308 107.937) (width 0.254) (layer B.Cu) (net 6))
 (segment (start 155.308 107.937) (end 155.308 104.94) (width 0.254) (layer B.Cu) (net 6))
 (segment (start 155.308 104.94) (end 153.454 103.086) (width 0.254) (layer B.Cu) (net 6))
 (segment (start 153.454 103.086) (end 153.454 102.502) (width 0.254) (layer B.Cu) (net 6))
 (segment (start 153.454 102.502) (end 153.124 102.172) (width 0.254) (layer B.Cu) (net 6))
 (segment (start 153.124 102.172) (end 153.098 102.172) (width 0.254) (layer B.Cu) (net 6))
 (via (at 153.098 102.172) (size 0.635) (layers F.Cu B.Cu) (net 6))
 (segment (start 148.908 98.7425) (end 148.908 100.774) (width 0.254) (layer F.Cu) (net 7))
 (segment (start 148.908 100.774) (end 149.542 101.41) (width 0.254) (layer F.Cu) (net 7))
 (segment (start 149.542 101.41) (end 151.956 101.41) (width 0.254) (layer F.Cu) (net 7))
 (segment (start 151.956 101.41) (end 152.006 101.41) (width 0.254) (layer B.Cu) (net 7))
 (segment (start 152.006 101.41) (end 152.413 101.816) (width 0.254) (layer B.Cu) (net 7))
 (segment (start 152.413 101.816) (end 152.413 102.832) (width 0.254) (layer B.Cu) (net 7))
 (segment (start 152.413 102.832) (end 154.8 105.22) (width 0.254) (layer B.Cu) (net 7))
 (segment (start 154.8 105.22) (end 154.8 108.115) (width 0.254) (layer B.Cu) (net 7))
 (segment (start 154.8 108.115) (end 155.838 109.152) (width 0.254) (layer B.Cu) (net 7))
 (segment (start 155.838 109.152) (end 156.782 109.152) (width 0.254) (layer B.Cu) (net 7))
 (via (at 151.956 101.41) (size 0.635) (layers F.Cu B.Cu) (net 7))
 (segment (start 119.316 100.074) (end 119.316 100.0735) (width 0.254) (layer F.Cu) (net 9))
 (segment (start 119.316 105.727) (end 119.316 100.074) (width 0.254) (layer F.Cu) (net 9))
 (segment (start 119.316 105.728) (end 119.316 105.727) (width 0.254) (layer F.Cu) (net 9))
 (segment (start 120.968 119.062) (end 113.778 119.062) (width 0.254) (layer F.Cu) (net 10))
 (segment (start 131 108.268) (end 131 105.904) (width 0.254) (layer F.Cu) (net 13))
 (segment (start 128.89 108.902) (end 130.366 108.902) (width 0.254) (layer F.Cu) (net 13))
 (segment (start 130.366 108.902) (end 131 108.268) (width 0.254) (layer F.Cu) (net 13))
 (segment (start 133.238 108.902) (end 131.636 108.902) (width 0.254) (layer F.Cu) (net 13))
 (segment (start 131.636 108.902) (end 131 108.268) (width 0.254) (layer F.Cu) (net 13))
 (segment (start 131 111.902) (end 131 108.268) (width 0.254) (layer F.Cu) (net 13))
 (segment (start 131 111.902) (end 127.62 111.902) (width 0.254) (layer F.Cu) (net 13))
 (segment (start 127.62 111.902) (end 126.512 113.01) (width 0.254) (layer F.Cu) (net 13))
 (segment (start 126.512 113.01) (end 126.512 116.142) (width 0.254) (layer F.Cu) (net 13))
 (segment (start 126.512 116.142) (end 129.476 116.142) (width 0.254) (layer F.Cu) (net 13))
 (segment (start 129.476 116.142) (end 130.238 116.904) (width 0.254) (layer F.Cu) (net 13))
 (segment (start 130.238 116.904) (end 133.032 116.904) (width 0.254) (layer F.Cu) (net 13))
 (segment (start 133.032 116.904) (end 133.668 117.538) (width 0.254) (layer F.Cu) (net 13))
 (segment (start 133.668 117.538) (end 133.668 119.062) (width 0.254) (layer F.Cu) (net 13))
 (segment (start 138.748 98.7425) (end 138.748 100.14) (width 0.254) (layer B.Cu) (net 24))
 (segment (start 138.748 100.14) (end 138.494 100.394) (width 0.254) (layer B.Cu) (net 24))
 (segment (start 138.494 100.394) (end 130.238 100.394) (width 0.254) (layer B.Cu) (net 24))
 (segment (start 130.238 100.394) (end 124.27 106.362) (width 0.254) (layer B.Cu) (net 24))
 (segment (start 124.27 106.362) (end 122.872 106.362) (width 0.254) (layer B.Cu) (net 24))
 (segment (start 122.872 106.362) (end 122.872 103.78) (width 0.254) (layer B.Cu) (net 24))
 (segment (start 141.288 98.7425) (end 141.288 100.648) (width 0.254) (layer B.Cu) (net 25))
 (segment (start 141.288 100.648) (end 141.034 100.902) (width 0.254) (layer B.Cu) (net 25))
 (segment (start 141.034 100.902) (end 130.492 100.902) (width 0.254) (layer B.Cu) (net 25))
 (segment (start 130.492 100.902) (end 128.46 102.934) (width 0.254) (layer B.Cu) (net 25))
 (segment (start 128.46 102.934) (end 128.46 107.294) (width 0.254) (layer B.Cu) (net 25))
 (segment (start 140.018 103.696) (end 140.018 107.802) (width 0.254) (layer B.Cu) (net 28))
 (segment (start 156.528 98.7425) (end 156.528 99.8855) (width 0.254) (layer B.Cu) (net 28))
 (segment (start 156.528 99.8855) (end 156.274 100.14) (width 0.254) (layer B.Cu) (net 28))
 (segment (start 156.274 100.14) (end 142.812 100.14) (width 0.254) (layer B.Cu) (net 28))
 (segment (start 142.812 100.14) (end 140.018 102.934) (width 0.254) (layer B.Cu) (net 28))
 (segment (start 140.018 102.934) (end 140.018 103.696) (width 0.254) (layer B.Cu) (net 28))
 (segment (start 140.018 103.696) (end 140.018 107.802) (width 0.254) (layer B.Cu) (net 28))
 (segment (start 133.102 107.638) (end 131.894 107.638) (width 0.254) (layer B.Cu) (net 28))
 (segment (start 131.894 107.638) (end 131.508 107.252) (width 0.254) (layer B.Cu) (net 28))
 (segment (start 131.508 107.252) (end 131.508 103.822) (width 0.254) (layer B.Cu) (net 28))
 (segment (start 131.508 103.822) (end 132.144 103.188) (width 0.254) (layer B.Cu) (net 28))
 (segment (start 132.144 103.188) (end 139.51 103.188) (width 0.254) (layer B.Cu) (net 28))
 (segment (start 139.51 103.188) (end 140.018 103.696) (width 0.254) (layer B.Cu) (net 28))
 (segment (start 159.068 98.7425) (end 159.068 100.012) (width 0.254) (layer B.Cu) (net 29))
 (segment (start 159.068 100.012) (end 158.432 100.648) (width 0.254) (layer B.Cu) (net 29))
 (segment (start 158.432 100.648) (end 143.32 100.648) (width 0.254) (layer B.Cu) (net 29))
 (segment (start 143.32 100.648) (end 143.002 100.965) (width 0.254) (layer B.Cu) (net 29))
 (segment (start 143.002 100.965) (end 142.812 101.156) (width 0.254) (layer B.Cu) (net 29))
 (segment (start 142.812 101.156) (end 142.812 101.664) (width 0.254) (layer B.Cu) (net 29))
 (segment (start 139.256 102.298) (end 132.27 102.298) (width 0.254) (layer B.Cu) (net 29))
 (segment (start 132.27 102.298) (end 131 103.568) (width 0.254) (layer B.Cu) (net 29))
 (segment (start 131 103.568) (end 131 107.76) (width 0.254) (layer B.Cu) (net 29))
 (segment (start 131 107.76) (end 131.828 108.588) (width 0.254) (layer B.Cu) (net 29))
 (segment (start 131.828 108.588) (end 133.102 108.588) (width 0.254) (layer B.Cu) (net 29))
 (segment (start 142.812 101.664) (end 142.176 102.298) (width 0.254) (layer F.Cu) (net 29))
 (segment (start 142.176 102.298) (end 139.256 102.298) (width 0.254) (layer F.Cu) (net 29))
 (segment (start 141.922 107.802) (end 141.922 102.552) (width 0.254) (layer B.Cu) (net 29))
 (segment (start 141.922 102.552) (end 142.812 101.664) (width 0.254) (layer B.Cu) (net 29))
 (via (at 139.256 102.298) (size 0.635) (layers F.Cu B.Cu) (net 29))
 (via (at 142.812 101.664) (size 0.635) (layers F.Cu B.Cu) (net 29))
 (segment (start 119.634 108.585) (end 119.316 108.268) (width 0.254) (layer B.Cu) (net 30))
 (segment (start 122.872 108.902) (end 119.952 108.902) (width 0.254) (layer B.Cu) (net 30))
 (segment (start 119.952 108.902) (end 119.634 108.585) (width 0.254) (layer B.Cu) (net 30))
 (segment (start 119.634 108.585) (end 119.316 108.267) (width 0.254) (layer B.Cu) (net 30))
 (segment (start 122.872 111.442) (end 125.794 111.442) (width 0.254) (layer B.Cu) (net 31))
 (segment (start 125.794 111.442) (end 128.334 113.982) (width 0.254) (layer B.Cu) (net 31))
 (segment (start 128.334 113.982) (end 133.922 113.982) (width 0.254) (layer B.Cu) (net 31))
 (segment (start 133.922 113.982) (end 134.302 113.602) (width 0.254) (layer B.Cu) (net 31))
 (segment (start 134.302 113.602) (end 134.302 109.03) (width 0.254) (layer B.Cu) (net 31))
 (segment (start 134.302 109.03) (end 134.744 108.588) (width 0.254) (layer B.Cu) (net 31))
 (segment (start 134.744 108.588) (end 135.502 108.588) (width 0.254) (layer B.Cu) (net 31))
 (segment (start 133.286 114.956) (end 131.346 114.956) (width 0.254) (layer F.Cu) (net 33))
 (segment (start 131.346 114.956) (end 131 115.302) (width 0.254) (layer F.Cu) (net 33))
 (segment (start 125.49 108.902) (end 125.49 107.216) (width 0.254) (layer F.Cu) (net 34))
 (segment (start 125.49 107.216) (end 126.09 106.616) (width 0.254) (layer F.Cu) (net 34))
 (segment (start 131 102.504) (end 132.686 102.504) (width 0.254) (layer F.Cu) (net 35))
 (segment (start 132.686 102.504) (end 133.286 103.104) (width 0.254) (layer F.Cu) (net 35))
 (segment (start 128.504 109.538) (end 128.46 109.494) (width 0.254) (layer B.Cu) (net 32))
 (segment (start 133.102 109.538) (end 128.504 109.538) (width 0.254) (layer B.Cu) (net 32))
 (segment (start 133.032 112.882) (end 133.032 109.608) (width 0.254) (layer B.Cu) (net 32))
 (segment (start 133.032 109.608) (end 133.102 109.538) (width 0.254) (layer B.Cu) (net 32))
 (segment (start 128.504 109.538) (end 128.46 109.494) (width 0.254) (layer B.Cu) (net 32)))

